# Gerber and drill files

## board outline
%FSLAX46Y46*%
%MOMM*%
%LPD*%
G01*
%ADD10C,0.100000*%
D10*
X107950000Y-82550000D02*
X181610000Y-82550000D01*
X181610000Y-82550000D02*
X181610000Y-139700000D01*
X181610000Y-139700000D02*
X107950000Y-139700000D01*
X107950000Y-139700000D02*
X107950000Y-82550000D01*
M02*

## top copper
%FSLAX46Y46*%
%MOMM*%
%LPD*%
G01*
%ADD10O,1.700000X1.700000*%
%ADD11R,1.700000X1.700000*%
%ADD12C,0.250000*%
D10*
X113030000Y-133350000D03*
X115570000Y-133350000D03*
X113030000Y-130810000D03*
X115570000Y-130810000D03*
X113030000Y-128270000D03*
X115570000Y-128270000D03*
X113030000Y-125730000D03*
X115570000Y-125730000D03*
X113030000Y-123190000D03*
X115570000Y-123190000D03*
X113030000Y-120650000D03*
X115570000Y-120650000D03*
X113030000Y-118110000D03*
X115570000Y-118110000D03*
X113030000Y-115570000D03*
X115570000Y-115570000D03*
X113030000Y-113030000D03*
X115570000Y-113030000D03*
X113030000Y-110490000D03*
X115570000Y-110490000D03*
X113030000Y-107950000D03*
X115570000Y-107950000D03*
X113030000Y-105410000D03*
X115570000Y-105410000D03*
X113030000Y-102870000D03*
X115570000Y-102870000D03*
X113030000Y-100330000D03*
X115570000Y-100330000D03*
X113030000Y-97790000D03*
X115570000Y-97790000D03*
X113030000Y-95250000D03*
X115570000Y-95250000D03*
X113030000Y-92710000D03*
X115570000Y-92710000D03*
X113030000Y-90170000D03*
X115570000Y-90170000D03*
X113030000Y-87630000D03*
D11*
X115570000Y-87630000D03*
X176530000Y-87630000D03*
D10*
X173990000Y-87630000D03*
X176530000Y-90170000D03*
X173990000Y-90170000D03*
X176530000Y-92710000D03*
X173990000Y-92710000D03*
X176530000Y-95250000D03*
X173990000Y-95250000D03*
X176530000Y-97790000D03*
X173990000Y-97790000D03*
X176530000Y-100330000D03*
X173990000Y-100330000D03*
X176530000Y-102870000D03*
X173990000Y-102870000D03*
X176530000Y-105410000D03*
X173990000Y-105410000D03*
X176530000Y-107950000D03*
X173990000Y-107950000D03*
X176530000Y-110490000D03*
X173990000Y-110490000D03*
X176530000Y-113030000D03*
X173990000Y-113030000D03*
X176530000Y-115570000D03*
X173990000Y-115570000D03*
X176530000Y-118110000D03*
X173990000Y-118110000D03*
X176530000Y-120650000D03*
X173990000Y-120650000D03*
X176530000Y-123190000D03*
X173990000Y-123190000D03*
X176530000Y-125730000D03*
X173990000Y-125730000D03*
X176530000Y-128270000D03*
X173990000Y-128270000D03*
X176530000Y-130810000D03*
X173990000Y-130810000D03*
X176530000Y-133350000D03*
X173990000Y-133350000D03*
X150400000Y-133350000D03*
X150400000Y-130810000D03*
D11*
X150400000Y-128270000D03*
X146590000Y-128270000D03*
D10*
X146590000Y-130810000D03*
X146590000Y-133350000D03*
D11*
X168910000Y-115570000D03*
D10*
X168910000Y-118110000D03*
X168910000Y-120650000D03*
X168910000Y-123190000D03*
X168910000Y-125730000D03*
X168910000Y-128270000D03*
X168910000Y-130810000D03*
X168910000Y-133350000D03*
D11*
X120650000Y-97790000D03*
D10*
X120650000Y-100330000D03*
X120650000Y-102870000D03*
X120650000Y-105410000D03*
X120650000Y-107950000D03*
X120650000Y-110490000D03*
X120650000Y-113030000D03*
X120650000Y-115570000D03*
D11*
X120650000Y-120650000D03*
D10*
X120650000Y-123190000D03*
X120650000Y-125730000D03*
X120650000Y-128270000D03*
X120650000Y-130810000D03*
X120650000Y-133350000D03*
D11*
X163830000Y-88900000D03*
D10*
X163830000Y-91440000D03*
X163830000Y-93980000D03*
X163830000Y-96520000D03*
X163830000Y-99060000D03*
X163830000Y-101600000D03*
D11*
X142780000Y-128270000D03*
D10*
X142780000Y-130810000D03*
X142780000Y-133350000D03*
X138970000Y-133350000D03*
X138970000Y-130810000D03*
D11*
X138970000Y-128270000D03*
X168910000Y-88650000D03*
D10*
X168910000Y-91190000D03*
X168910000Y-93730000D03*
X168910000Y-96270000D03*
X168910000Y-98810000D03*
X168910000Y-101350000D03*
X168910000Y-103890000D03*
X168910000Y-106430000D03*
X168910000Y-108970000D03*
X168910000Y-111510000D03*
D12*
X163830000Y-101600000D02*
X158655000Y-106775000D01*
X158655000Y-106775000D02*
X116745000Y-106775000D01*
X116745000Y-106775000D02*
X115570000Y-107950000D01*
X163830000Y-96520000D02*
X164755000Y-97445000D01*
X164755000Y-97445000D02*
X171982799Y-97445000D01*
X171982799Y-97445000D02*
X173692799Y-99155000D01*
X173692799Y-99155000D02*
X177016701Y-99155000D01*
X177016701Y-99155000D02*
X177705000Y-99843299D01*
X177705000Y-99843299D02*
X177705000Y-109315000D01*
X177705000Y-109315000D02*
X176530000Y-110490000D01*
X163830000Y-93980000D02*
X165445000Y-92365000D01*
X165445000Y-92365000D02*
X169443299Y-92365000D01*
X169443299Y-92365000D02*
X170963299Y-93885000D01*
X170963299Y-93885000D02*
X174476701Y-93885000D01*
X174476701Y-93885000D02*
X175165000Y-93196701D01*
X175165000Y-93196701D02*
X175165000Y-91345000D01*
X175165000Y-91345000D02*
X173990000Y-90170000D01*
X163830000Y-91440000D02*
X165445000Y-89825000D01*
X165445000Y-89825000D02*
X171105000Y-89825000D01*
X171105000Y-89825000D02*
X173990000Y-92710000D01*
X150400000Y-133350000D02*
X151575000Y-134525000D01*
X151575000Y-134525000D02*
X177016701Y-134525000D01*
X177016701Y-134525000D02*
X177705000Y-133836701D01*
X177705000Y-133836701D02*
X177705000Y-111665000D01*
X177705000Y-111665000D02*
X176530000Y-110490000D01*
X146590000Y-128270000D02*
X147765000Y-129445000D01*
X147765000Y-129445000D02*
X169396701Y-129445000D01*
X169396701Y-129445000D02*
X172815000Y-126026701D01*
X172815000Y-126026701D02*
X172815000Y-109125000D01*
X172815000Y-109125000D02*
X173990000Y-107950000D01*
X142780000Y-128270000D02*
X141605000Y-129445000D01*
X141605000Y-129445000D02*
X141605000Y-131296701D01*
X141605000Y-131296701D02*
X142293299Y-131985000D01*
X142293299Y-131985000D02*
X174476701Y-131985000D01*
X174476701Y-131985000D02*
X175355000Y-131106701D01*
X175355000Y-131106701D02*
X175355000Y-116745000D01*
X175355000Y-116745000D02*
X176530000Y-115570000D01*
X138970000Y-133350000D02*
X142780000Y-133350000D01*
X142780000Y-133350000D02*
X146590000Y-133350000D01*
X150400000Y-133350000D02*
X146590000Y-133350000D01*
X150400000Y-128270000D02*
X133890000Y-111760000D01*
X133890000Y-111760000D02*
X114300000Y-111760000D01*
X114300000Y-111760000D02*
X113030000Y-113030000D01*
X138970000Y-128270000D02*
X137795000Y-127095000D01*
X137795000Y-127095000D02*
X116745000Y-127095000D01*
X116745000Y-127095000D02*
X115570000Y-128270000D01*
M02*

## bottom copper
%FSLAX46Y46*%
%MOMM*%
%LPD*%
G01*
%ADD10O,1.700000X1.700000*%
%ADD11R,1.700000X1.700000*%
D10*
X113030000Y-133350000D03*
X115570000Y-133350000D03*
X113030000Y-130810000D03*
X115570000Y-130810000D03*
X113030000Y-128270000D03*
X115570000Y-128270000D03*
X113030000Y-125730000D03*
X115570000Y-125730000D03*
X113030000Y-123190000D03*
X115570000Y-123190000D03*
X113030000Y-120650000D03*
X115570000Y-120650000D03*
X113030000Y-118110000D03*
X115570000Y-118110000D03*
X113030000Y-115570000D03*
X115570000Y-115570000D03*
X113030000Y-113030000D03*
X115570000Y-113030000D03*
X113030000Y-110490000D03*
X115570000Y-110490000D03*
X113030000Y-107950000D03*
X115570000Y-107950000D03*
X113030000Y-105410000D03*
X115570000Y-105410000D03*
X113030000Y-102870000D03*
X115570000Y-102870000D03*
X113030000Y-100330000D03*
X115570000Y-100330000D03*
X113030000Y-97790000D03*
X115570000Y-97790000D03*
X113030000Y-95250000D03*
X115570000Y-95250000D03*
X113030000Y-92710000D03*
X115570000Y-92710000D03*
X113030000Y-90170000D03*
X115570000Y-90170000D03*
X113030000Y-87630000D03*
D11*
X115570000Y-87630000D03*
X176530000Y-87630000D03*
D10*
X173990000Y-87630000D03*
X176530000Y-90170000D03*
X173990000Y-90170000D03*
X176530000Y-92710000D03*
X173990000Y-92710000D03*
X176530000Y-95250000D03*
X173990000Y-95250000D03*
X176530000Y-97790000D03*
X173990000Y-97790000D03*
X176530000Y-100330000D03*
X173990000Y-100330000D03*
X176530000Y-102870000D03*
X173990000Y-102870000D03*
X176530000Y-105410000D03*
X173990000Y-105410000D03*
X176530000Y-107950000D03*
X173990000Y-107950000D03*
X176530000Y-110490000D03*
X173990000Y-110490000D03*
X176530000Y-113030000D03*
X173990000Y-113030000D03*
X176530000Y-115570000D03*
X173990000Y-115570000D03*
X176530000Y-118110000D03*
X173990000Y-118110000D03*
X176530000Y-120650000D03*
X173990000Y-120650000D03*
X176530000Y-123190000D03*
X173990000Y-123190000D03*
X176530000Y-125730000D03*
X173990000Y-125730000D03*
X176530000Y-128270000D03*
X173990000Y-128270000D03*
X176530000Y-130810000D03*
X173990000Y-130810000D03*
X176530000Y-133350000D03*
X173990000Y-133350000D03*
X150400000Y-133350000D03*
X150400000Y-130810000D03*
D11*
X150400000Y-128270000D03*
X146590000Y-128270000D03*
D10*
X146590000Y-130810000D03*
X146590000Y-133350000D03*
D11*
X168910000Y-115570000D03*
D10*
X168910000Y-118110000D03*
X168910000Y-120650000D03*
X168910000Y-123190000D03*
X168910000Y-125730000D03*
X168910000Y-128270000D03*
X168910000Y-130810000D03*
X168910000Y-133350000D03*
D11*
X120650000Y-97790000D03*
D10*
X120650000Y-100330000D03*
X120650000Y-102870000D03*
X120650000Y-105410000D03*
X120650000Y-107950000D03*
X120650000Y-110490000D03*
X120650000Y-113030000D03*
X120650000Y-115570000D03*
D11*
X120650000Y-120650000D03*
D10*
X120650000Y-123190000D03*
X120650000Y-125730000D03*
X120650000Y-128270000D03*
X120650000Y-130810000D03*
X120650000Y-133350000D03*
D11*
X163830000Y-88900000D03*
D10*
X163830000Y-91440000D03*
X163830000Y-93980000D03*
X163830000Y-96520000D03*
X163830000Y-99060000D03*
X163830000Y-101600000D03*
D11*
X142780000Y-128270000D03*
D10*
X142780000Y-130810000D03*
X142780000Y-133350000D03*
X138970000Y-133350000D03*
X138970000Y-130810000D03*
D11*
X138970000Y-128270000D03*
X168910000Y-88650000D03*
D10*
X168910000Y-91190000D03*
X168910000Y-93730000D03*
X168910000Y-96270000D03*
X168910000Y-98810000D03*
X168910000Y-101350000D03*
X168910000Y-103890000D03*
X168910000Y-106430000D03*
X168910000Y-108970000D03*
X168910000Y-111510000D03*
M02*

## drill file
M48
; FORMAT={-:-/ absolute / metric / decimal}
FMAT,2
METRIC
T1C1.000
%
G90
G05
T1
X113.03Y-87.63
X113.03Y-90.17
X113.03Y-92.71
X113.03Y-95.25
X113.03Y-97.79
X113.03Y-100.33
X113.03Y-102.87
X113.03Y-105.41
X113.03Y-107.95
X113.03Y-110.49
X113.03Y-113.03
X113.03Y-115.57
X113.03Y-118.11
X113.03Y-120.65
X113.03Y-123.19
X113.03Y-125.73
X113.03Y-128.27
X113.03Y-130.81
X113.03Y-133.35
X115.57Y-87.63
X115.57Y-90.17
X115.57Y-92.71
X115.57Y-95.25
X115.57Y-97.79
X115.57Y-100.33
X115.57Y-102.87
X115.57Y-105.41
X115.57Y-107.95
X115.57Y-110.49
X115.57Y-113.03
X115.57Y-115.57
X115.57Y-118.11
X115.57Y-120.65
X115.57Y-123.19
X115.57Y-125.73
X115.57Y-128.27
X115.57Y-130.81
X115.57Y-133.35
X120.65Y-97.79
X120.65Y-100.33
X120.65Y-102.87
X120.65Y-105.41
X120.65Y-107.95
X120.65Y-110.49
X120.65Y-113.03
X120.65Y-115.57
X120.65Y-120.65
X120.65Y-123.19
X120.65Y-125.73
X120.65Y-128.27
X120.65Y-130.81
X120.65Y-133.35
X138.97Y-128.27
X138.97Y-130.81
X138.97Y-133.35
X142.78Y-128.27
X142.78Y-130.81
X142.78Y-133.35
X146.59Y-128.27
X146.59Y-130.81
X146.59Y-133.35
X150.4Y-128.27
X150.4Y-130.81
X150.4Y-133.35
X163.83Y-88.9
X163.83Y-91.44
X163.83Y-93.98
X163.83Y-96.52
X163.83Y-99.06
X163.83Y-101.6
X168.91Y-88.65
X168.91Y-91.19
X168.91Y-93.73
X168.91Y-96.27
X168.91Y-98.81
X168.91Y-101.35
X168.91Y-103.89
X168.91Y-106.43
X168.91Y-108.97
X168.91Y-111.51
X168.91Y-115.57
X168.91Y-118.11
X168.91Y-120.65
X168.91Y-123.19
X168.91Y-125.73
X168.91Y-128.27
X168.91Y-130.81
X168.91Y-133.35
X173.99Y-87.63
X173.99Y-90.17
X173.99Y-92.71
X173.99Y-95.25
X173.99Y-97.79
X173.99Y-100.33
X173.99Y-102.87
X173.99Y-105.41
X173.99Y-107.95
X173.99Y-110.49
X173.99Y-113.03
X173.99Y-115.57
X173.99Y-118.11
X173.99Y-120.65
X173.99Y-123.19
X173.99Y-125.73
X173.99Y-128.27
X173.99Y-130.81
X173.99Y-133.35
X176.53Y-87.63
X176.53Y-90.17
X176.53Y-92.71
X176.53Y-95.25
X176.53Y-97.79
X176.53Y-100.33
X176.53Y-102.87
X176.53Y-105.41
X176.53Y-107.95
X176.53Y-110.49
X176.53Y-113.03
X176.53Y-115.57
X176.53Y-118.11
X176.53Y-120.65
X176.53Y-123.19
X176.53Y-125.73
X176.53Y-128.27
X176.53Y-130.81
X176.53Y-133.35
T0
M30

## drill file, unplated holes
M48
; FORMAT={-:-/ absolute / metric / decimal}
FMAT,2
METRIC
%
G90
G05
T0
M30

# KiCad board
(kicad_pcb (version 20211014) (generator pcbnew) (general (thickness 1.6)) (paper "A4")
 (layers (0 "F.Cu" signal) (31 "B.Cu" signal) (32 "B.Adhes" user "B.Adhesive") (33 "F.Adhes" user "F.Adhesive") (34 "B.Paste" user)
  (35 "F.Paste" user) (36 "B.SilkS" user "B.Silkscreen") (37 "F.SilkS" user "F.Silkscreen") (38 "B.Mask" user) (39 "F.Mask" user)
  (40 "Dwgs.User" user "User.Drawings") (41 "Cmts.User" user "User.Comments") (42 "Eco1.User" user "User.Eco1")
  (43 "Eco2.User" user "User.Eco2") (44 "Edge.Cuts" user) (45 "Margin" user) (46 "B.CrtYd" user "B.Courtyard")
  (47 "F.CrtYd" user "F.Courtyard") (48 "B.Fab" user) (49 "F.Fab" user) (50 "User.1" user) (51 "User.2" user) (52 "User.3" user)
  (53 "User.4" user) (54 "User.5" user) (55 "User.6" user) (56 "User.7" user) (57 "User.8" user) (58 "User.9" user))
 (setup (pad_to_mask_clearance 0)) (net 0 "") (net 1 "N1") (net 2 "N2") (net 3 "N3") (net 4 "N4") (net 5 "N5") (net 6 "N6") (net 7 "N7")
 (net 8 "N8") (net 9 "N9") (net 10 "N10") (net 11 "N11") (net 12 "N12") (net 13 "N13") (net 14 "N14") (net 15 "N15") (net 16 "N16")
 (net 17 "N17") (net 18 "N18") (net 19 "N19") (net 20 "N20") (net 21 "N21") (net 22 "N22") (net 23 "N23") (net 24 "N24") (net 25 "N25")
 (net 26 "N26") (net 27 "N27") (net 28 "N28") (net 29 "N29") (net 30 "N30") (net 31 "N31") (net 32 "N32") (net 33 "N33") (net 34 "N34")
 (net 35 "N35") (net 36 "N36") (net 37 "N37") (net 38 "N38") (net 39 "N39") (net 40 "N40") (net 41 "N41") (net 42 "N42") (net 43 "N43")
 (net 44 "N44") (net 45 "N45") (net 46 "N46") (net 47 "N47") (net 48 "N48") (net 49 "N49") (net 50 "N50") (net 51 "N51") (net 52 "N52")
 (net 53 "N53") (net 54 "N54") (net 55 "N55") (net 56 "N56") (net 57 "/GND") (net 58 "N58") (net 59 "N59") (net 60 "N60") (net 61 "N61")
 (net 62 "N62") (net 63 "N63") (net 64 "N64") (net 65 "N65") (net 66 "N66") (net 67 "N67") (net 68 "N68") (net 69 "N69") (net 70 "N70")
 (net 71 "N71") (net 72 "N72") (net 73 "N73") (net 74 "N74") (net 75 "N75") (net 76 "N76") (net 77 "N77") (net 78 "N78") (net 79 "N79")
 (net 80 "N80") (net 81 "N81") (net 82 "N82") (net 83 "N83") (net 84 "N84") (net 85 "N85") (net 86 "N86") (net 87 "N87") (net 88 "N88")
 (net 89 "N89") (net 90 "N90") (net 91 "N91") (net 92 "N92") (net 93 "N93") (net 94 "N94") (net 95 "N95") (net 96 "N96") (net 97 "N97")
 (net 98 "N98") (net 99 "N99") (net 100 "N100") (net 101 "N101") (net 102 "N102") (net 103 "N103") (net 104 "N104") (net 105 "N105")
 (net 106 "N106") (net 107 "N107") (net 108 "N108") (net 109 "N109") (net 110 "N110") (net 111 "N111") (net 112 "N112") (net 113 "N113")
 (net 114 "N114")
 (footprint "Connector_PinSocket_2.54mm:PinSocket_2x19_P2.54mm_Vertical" (layer "F.Cu") (at 115.57 87.63)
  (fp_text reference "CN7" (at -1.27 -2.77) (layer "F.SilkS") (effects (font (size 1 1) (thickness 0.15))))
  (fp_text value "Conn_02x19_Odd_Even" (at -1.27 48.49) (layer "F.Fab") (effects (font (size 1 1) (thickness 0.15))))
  (pad "1" thru_hole rect locked (at 0 0) (size 1.7 1.7) (drill 1) (layers *.Cu *.Mask) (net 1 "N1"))
  (pad "2" thru_hole oval locked (at -2.54 0) (size 1.7 1.7) (drill 1) (layers *.Cu *.Mask) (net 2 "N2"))
  (pad "3" thru_hole oval locked (at 0 2.54) (size 1.7 1.7) (drill 1) (layers *.Cu *.Mask) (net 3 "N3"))
  (pad "4" thru_hole oval locked (at -2.54 2.54) (size 1.7 1.7) (drill 1) (layers *.Cu *.Mask) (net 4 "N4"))
  (pad "5" thru_hole oval locked (at 0 5.08) (size 1.7 1.7) (drill 1) (layers *.Cu *.Mask) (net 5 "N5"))
  (pad "6" thru_hole oval locked (at -2.54 5.08) (size 1.7 1.7) (drill 1) (layers *.Cu *.Mask) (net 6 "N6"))
  (pad "7" thru_hole oval locked (at 0 7.62) (size 1.7 1.7) (drill 1) (layers *.Cu *.Mask) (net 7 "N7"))
  (pad "8" thru_hole oval locked (at -2.54 7.62) (size 1.7 1.7) (drill 1) (layers *.Cu *.Mask) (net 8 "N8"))
  (pad "9" thru_hole oval locked (at 0 10.16) (size 1.7 1.7) (drill 1) (layers *.Cu *.Mask) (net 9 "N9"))
  (pad "10" thru_hole oval locked (at -2.54 10.16) (size 1.7 1.7) (drill 1) (layers *.Cu *.Mask) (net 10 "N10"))
  (pad "11" thru_hole oval locked (at 0 12.7) (size 1.7 1.7) (drill 1) (layers *.Cu *.Mask) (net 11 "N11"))
  (pad "12" thru_hole oval locked (at -2.54 12.7) (size 1.7 1.7) (drill 1) (layers *.Cu *.Mask) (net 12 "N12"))
  (pad "13" thru_hole oval locked (at 0 15.24) (size 1.7 1.7) (drill 1) (layers *.Cu *.Mask) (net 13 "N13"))
  (pad "14" thru_hole oval locked (at -2.54 15.24) (size 1.7 1.7) (drill 1) (layers *.Cu *.Mask) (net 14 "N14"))
  (pad "15" thru_hole oval locked (at 0 17.78) (size 1.7 1.7) (drill 1) (layers *.Cu *.Mask) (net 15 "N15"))
  (pad "16" thru_hole oval locked (at -2.54 17.78) (size 1.7 1.7) (drill 1) (layers *.Cu *.Mask) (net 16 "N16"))
  (pad "17" thru_hole oval locked (at 0 20.32) (size 1.7 1.7) (drill 1) (layers *.Cu *.Mask) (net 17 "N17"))
  (pad "18" thru_hole oval locked (at -2.54 20.32) (size 1.7 1.7) (drill 1) (layers *.Cu *.Mask) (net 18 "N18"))
  (pad "19" thru_hole oval locked (at 0 22.86) (size 1.7 1.7) (drill 1) (layers *.Cu *.Mask) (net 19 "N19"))
  (pad "20" thru_hole oval locked (at -2.54 22.86) (size 1.7 1.7) (drill 1) (layers *.Cu *.Mask) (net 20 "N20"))
  (pad "21" thru_hole oval locked (at 0 25.4) (size 1.7 1.7) (drill 1) (layers *.Cu *.Mask) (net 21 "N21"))
  (pad "22" thru_hole oval locked (at -2.54 25.4) (size 1.7 1.7) (drill 1) (layers *.Cu *.Mask) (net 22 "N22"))
  (pad "23" thru_hole oval locked (at 0 27.94) (size 1.7 1.7) (drill 1) (layers *.Cu *.Mask) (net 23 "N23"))
  (pad "24" thru_hole oval locked (at -2.54 27.94) (size 1.7 1.7) (drill 1) (layers *.Cu *.Mask) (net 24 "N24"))
  (pad "25" thru_hole oval locked (at 0 30.48) (size 1.7 1.7) (drill 1) (layers *.Cu *.Mask) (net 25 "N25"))
  (pad "26" thru_hole oval locked (at -2.54 30.48) (size 1.7 1.7) (drill 1) (layers *.Cu *.Mask) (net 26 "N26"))
  (pad "27" thru_hole oval locked (at 0 33.02) (size 1.7 1.7) (drill 1) (layers *.Cu *.Mask) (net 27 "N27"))
  (pad "28" thru_hole oval locked (at -2.54 33.02) (size 1.7 1.7) (drill 1) (layers *.Cu *.Mask) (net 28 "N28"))
  (pad "29" thru_hole oval locked (at 0 35.56) (size 1.7 1.7) (drill 1) (layers *.Cu *.Mask) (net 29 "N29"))
  (pad "30" thru_hole oval locked (at -2.54 35.56) (size 1.7 1.7) (drill 1) (layers *.Cu *.Mask) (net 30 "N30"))
  (pad "31" thru_hole oval locked (at 0 38.1) (size 1.7 1.7) (drill 1) (layers *.Cu *.Mask) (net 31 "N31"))
  (pad "32" thru_hole oval locked (at -2.54 38.1) (size 1.7 1.7) (drill 1) (layers *.Cu *.Mask) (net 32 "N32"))
  (pad "33" thru_hole oval locked (at 0 40.64) (size 1.7 1.7) (drill 1) (layers *.Cu *.Mask) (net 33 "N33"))
  (pad "34" thru_hole oval locked (at -2.54 40.64) (size 1.7 1.7) (drill 1) (layers *.Cu *.Mask) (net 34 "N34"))
  (pad "35" thru_hole oval locked (at 0 43.18) (size 1.7 1.7) (drill 1) (layers *.Cu *.Mask) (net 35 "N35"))
  (pad "36" thru_hole oval locked (at -2.54 43.18) (size 1.7 1.7) (drill 1) (layers *.Cu *.Mask) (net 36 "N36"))
  (pad "37" thru_hole oval locked (at 0 45.72) (size 1.7 1.7) (drill 1) (layers *.Cu *.Mask) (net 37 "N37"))
  (pad "38" thru_hole oval locked (at -2.54 45.72) (size 1.7 1.7) (drill 1) (layers *.Cu *.Mask) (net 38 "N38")))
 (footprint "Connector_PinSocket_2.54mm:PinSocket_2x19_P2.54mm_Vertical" (layer "F.Cu") (at 176.53 87.63)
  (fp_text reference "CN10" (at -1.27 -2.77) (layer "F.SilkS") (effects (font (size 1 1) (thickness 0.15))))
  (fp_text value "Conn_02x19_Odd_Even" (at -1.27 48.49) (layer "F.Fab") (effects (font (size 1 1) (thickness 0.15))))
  (pad "1" thru_hole rect (at 0 0) (size 1.7 1.7) (drill 1) (layers *.Cu *.Mask) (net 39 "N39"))
  (pad "2" thru_hole oval (at -2.54 0) (size 1.7 1.7) (drill 1) (layers *.Cu *.Mask) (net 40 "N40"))
  (pad "3" thru_hole oval (at 0 2.54) (size 1.7 1.7) (drill 1) (layers *.Cu *.Mask) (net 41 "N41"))
  (pad "4" thru_hole oval (at -2.54 2.54) (size 1.7 1.7) (drill 1) (layers *.Cu *.Mask) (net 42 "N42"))
  (pad "5" thru_hole oval (at 0 5.08) (size 1.7 1.7) (drill 1) (layers *.Cu *.Mask) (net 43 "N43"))
  (pad "6" thru_hole oval (at -2.54 5.08) (size 1.7 1.7) (drill 1) (layers *.Cu *.Mask) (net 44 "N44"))
  (pad "7" thru_hole oval (at 0 7.62) (size 1.7 1.7) (drill 1) (layers *.Cu *.Mask) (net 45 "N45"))
  (pad "8" thru_hole oval (at -2.54 7.62) (size 1.7 1.7) (drill 1) (layers *.Cu *.Mask) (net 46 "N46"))
  (pad "9" thru_hole oval (at 0 10.16) (size 1.7 1.7) (drill 1) (layers *.Cu *.Mask) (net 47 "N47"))
  (pad "10" thru_hole oval (at -2.54 10.16) (size 1.7 1.7) (drill 1) (layers *.Cu *.Mask) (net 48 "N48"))
  (pad "11" thru_hole oval (at 0 12.7) (size 1.7 1.7) (drill 1) (layers *.Cu *.Mask) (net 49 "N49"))
  (pad "12" thru_hole oval (at -2.54 12.7) (size 1.7 1.7) (drill 1) (layers *.Cu *.Mask) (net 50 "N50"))
  (pad "13" thru_hole oval (at 0 15.24) (size 1.7 1.7) (drill 1) (layers *.Cu *.Mask) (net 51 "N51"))
  (pad "14" thru_hole oval (at -2.54 15.24) (size 1.7 1.7) (drill 1) (layers *.Cu *.Mask) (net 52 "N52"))
  (pad "15" thru_hole oval (at 0 17.78) (size 1.7 1.7) (drill 1) (layers *.Cu *.Mask) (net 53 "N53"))
  (pad "16" thru_hole oval (at -2.54 17.78) (size 1.7 1.7) (drill 1) (layers *.Cu *.Mask) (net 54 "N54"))
  (pad "17" thru_hole oval (at 0 20.32) (size 1.7 1.7) (drill 1) (layers *.Cu *.Mask) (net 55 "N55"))
  (pad "18" thru_hole oval (at -2.54 20.32) (size 1.7 1.7) (drill 1) (layers *.Cu *.Mask) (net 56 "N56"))
  (pad "19" thru_hole oval (at 0 22.86) (size 1.7 1.7) (drill 1) (layers *.Cu *.Mask) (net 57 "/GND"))
  (pad "20" thru_hole oval (at -2.54 22.86) (size 1.7 1.7) (drill 1) (layers *.Cu *.Mask) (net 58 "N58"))
  (pad "21" thru_hole oval (at 0 25.4) (size 1.7 1.7) (drill 1) (layers *.Cu *.Mask) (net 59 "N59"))
  (pad "22" thru_hole oval (at -2.54 25.4) (size 1.7 1.7) (drill 1) (layers *.Cu *.Mask) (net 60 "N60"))
  (pad "23" thru_hole oval (at 0 27.94) (size 1.7 1.7) (drill 1) (layers *.Cu *.Mask) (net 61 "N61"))
  (pad "24" thru_hole oval (at -2.54 27.94) (size 1.7 1.7) (drill 1) (layers *.Cu *.Mask) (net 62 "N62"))
  (pad "25" thru_hole oval (at 0 30.48) (size 1.7 1.7) (drill 1) (layers *.Cu *.Mask) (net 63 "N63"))
  (pad "26" thru_hole oval (at -2.54 30.48) (size 1.7 1.7) (drill 1) (layers *.Cu *.Mask) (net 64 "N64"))
  (pad "27" thru_hole oval (at 0 33.02) (size 1.7 1.7) (drill 1) (layers *.Cu *.Mask) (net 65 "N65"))
  (pad "28" thru_hole oval (at -2.54 33.02) (size 1.7 1.7) (drill 1) (layers *.Cu *.Mask) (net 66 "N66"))
  (pad "29" thru_hole oval (at 0 35.56) (size 1.7 1.7) (drill 1) (layers *.Cu *.Mask) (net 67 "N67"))
  (pad "30" thru_hole oval (at -2.54 35.56) (size 1.7 1.7) (drill 1) (layers *.Cu *.Mask) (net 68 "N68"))
  (pad "31" thru_hole oval (at 0 38.1) (size 1.7 1.7) (drill 1) (layers *.Cu *.Mask) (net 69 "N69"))
  (pad "32" thru_hole oval (at -2.54 38.1) (size 1.7 1.7) (drill 1) (layers *.Cu *.Mask) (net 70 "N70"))
  (pad "33" thru_hole oval (at 0 40.64) (size 1.7 1.7) (drill 1) (layers *.Cu *.Mask) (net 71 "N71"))
  (pad "34" thru_hole oval (at -2.54 40.64) (size 1.7 1.7) (drill 1) (layers *.Cu *.Mask) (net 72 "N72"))
  (pad "35" thru_hole oval (at 0 43.18) (size 1.7 1.7) (drill 1) (layers *.Cu *.Mask) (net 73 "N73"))
  (pad "36" thru_hole oval (at -2.54 43.18) (size 1.7 1.7) (drill 1) (layers *.Cu *.Mask) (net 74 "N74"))
  (pad "37" thru_hole oval (at 0 45.72) (size 1.7 1.7) (drill 1) (layers *.Cu *.Mask) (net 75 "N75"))
  (pad "38" thru_hole oval (at -2.54 45.72) (size 1.7 1.7) (drill 1) (layers *.Cu *.Mask) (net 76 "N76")))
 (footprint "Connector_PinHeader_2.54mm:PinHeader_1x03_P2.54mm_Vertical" (layer "F.Cu") (at 150.4 128.27)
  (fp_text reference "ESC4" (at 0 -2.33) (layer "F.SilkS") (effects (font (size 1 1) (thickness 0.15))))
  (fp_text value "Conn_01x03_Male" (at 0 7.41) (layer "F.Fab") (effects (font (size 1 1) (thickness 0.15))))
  (pad "1" thru_hole rect (at 0 0) (size 1.7 1.7) (drill 1) (layers *.Cu *.Mask) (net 22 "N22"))
  (pad "2" thru_hole oval (at 0 2.54) (size 1.7 1.7) (drill 1) (layers *.Cu *.Mask) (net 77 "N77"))
  (pad "3" thru_hole oval (at 0 5.08) (size 1.7 1.7) (drill 1) (layers *.Cu *.Mask) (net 57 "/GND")))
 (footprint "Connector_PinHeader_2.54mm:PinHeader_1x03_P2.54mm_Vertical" (layer "F.Cu") (at 146.59 128.27)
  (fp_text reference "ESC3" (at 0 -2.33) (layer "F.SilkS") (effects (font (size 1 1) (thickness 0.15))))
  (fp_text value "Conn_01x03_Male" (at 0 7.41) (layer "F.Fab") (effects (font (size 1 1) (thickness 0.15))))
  (pad "1" thru_hole rect (at 0 0) (size 1.7 1.7) (drill 1) (layers *.Cu *.Mask) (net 56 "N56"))
  (pad "2" thru_hole oval (at 0 2.54) (size 1.7 1.7) (drill 1) (layers *.Cu *.Mask) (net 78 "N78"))
  (pad "3" thru_hole oval (at 0 5.08) (size 1.7 1.7) (drill 1) (layers *.Cu *.Mask) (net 57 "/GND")))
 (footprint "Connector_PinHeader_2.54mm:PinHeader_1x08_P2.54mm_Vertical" (layer "F.Cu") (at 168.91 115.57)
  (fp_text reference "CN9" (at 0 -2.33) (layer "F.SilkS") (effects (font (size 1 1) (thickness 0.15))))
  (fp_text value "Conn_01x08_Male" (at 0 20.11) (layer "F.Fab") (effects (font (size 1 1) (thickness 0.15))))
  (pad "1" thru_hole rect (at 0 0) (size 1.7 1.7) (drill 1) (layers *.Cu *.Mask) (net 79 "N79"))
  (pad "2" thru_hole oval (at 0 2.54) (size 1.7 1.7) (drill 1) (layers *.Cu *.Mask) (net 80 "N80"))
  (pad "3" thru_hole oval (at 0 5.08) (size 1.7 1.7) (drill 1) (layers *.Cu *.Mask) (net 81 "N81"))
  (pad "4" thru_hole oval (at 0 7.62) (size 1.7 1.7) (drill 1) (layers *.Cu *.Mask) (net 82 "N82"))
  (pad "5" thru_hole oval (at 0 10.16) (size 1.7 1.7) (drill 1) (layers *.Cu *.Mask) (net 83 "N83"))
  (pad "6" thru_hole oval (at 0 12.7) (size 1.7 1.7) (drill 1) (layers *.Cu *.Mask) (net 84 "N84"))
  (pad "7" thru_hole oval (at 0 15.24) (size 1.7 1.7) (drill 1) (layers *.Cu *.Mask) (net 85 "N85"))
  (pad "8" thru_hole oval (at 0 17.78) (size 1.7 1.7) (drill 1) (layers *.Cu *.Mask) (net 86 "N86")))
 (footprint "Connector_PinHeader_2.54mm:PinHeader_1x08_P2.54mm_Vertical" (layer "F.Cu") (at 120.65 97.79)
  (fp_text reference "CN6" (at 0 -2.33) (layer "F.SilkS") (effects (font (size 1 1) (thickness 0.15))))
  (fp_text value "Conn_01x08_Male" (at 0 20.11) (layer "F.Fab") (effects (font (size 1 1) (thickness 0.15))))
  (pad "1" thru_hole rect (at 0 0) (size 1.7 1.7) (drill 1) (layers *.Cu *.Mask) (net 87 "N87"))
  (pad "2" thru_hole oval (at 0 2.54) (size 1.7 1.7) (drill 1) (layers *.Cu *.Mask) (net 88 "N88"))
  (pad "3" thru_hole oval (at 0 5.08) (size 1.7 1.7) (drill 1) (layers *.Cu *.Mask) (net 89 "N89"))
  (pad "4" thru_hole oval (at 0 7.62) (size 1.7 1.7) (drill 1) (layers *.Cu *.Mask) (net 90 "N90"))
  (pad "5" thru_hole oval (at 0 10.16) (size 1.7 1.7) (drill 1) (layers *.Cu *.Mask) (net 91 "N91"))
  (pad "6" thru_hole oval (at 0 12.7) (size 1.7 1.7) (drill 1) (layers *.Cu *.Mask) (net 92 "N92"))
  (pad "7" thru_hole oval (at 0 15.24) (size 1.7 1.7) (drill 1) (layers *.Cu *.Mask) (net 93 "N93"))
  (pad "8" thru_hole oval (at 0 17.78) (size 1.7 1.7) (drill 1) (layers *.Cu *.Mask) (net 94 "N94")))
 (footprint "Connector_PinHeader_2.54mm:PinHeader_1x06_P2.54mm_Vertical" (layer "F.Cu") (at 120.65 120.65)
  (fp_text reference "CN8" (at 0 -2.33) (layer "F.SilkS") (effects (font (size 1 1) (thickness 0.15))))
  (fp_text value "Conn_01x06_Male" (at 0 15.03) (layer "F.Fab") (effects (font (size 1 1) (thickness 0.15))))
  (pad "1" thru_hole rect (at 0 0) (size 1.7 1.7) (drill 1) (layers *.Cu *.Mask) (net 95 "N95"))
  (pad "2" thru_hole oval (at 0 2.54) (size 1.7 1.7) (drill 1) (layers *.Cu *.Mask) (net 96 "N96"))
  (pad "3" thru_hole oval (at 0 5.08) (size 1.7 1.7) (drill 1) (layers *.Cu *.Mask) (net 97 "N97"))
  (pad "4" thru_hole oval (at 0 7.62) (size 1.7 1.7) (drill 1) (layers *.Cu *.Mask) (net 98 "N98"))
  (pad "5" thru_hole oval (at 0 10.16) (size 1.7 1.7) (drill 1) (layers *.Cu *.Mask) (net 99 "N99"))
  (pad "6" thru_hole oval (at 0 12.7) (size 1.7 1.7) (drill 1) (layers *.Cu *.Mask) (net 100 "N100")))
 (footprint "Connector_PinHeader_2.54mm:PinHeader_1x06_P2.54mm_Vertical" (layer "F.Cu") (at 163.83 88.9)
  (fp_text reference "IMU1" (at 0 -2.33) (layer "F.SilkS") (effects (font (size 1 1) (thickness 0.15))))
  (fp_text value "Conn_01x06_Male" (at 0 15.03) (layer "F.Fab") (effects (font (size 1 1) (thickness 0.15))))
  (pad "1" thru_hole rect (at 0 0) (size 1.7 1.7) (drill 1) (layers *.Cu *.Mask) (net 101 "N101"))
  (pad "2" thru_hole oval (at 0 2.54) (size 1.7 1.7) (drill 1) (layers *.Cu *.Mask) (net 44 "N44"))
  (pad "3" thru_hole oval (at 0 5.08) (size 1.7 1.7) (drill 1) (layers *.Cu *.Mask) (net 42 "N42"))
  (pad "4" thru_hole oval (at 0 7.62) (size 1.7 1.7) (drill 1) (layers *.Cu *.Mask) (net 57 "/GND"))
  (pad "5" thru_hole oval (at 0 10.16) (size 1.7 1.7) (drill 1) (layers *.Cu *.Mask) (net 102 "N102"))
  (pad "6" thru_hole oval (at 0 12.7) (size 1.7 1.7) (drill 1) (layers *.Cu *.Mask) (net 17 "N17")))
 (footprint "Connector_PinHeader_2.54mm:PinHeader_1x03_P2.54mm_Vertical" (layer "F.Cu") (at 142.78 128.27)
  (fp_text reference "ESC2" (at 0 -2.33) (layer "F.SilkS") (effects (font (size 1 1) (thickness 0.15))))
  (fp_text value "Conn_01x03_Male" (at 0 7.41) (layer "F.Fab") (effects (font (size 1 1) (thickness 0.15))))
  (pad "1" thru_hole rect (at 0 0) (size 1.7 1.7) (drill 1) (layers *.Cu *.Mask) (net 61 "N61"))
  (pad "2" thru_hole oval (at 0 2.54) (size 1.7 1.7) (drill 1) (layers *.Cu *.Mask) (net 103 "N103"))
  (pad "3" thru_hole oval (at 0 5.08) (size 1.7 1.7) (drill 1) (layers *.Cu *.Mask) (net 57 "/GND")))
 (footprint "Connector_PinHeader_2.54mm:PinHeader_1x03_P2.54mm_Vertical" (layer "F.Cu") (at 138.97 128.27)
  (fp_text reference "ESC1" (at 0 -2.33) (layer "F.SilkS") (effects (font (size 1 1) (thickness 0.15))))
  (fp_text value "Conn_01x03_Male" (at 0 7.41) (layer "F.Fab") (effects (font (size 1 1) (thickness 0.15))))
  (pad "1" thru_hole rect (at 0 0) (size 1.7 1.7) (drill 1) (layers *.Cu *.Mask) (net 33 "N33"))
  (pad "2" thru_hole oval (at 0 2.54) (size 1.7 1.7) (drill 1) (layers *.Cu *.Mask) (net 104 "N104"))
  (pad "3" thru_hole oval (at 0 5.08) (size 1.7 1.7) (drill 1) (layers *.Cu *.Mask) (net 57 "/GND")))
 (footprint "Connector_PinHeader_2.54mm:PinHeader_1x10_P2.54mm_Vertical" (layer "F.Cu") (at 168.91 88.65)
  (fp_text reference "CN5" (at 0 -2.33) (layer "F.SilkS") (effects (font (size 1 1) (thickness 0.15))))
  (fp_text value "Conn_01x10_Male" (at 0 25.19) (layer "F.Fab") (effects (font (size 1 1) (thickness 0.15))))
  (pad "1" thru_hole rect (at 0 0) (size 1.7 1.7) (drill 1) (layers *.Cu *.Mask) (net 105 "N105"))
  (pad "2" thru_hole oval (at 0 2.54) (size 1.7 1.7) (drill 1) (layers *.Cu *.Mask) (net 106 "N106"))
  (pad "3" thru_hole oval (at 0 5.08) (size 1.7 1.7) (drill 1) (layers *.Cu *.Mask) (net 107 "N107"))
  (pad "4" thru_hole oval (at 0 7.62) (size 1.7 1.7) (drill 1) (layers *.Cu *.Mask) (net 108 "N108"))
  (pad "5" thru_hole oval (at 0 10.16) (size 1.7 1.7) (drill 1) (layers *.Cu *.Mask) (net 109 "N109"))
  (pad "6" thru_hole oval (at 0 12.7) (size 1.7 1.7) (drill 1) (layers *.Cu *.Mask) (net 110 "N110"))
  (pad "7" thru_hole oval (at 0 15.24) (size 1.7 1.7) (drill 1) (layers *.Cu *.Mask) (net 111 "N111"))
  (pad "8" thru_hole oval (at 0 17.78) (size 1.7 1.7) (drill 1) (layers *.Cu *.Mask) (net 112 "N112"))
  (pad "9" thru_hole oval (at 0 20.32) (size 1.7 1.7) (drill 1) (layers *.Cu *.Mask) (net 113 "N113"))
  (pad "10" thru_hole oval (at 0 22.86) (size 1.7 1.7) (drill 1) (layers *.Cu *.Mask) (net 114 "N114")))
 (gr_rect (start 107.95 82.55) (end 181.61 139.7) (layer "Edge.Cuts") (width 0.1) (fill none))
 (segment (start 133.89 111.76) (end 114.3 111.76) (width 0.25) (layer "F.Cu") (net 22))
 (segment (start 150.4 128.27) (end 133.89 111.76) (width 0.25) (layer "F.Cu") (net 22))
 (segment (start 114.3 111.76) (end 113.03 113.03) (width 0.25) (layer "F.Cu") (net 22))
 (segment (start 177.016701 99.155) (end 177.705 99.843299) (width 0.25) (layer "F.Cu") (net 57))
 (segment (start 177.705 99.843299) (end 177.705 109.315) (width 0.25) (layer "F.Cu") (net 57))
 (segment (start 177.705 111.665) (end 176.53 110.49) (width 0.25) (layer "F.Cu") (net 57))
 (segment (start 138.97 133.35) (end 142.78 133.35) (width 0.25) (layer "F.Cu") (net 57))
 (segment (start 173.692799 99.155) (end 177.016701 99.155) (width 0.25) (layer "F.Cu") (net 57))
 (segment (start 150.4 133.35) (end 151.575 134.525) (width 0.25) (layer "F.Cu") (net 57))
 (segment (start 177.705 109.315) (end 176.53 110.49) (width 0.25) (layer "F.Cu") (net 57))
 (segment (start 150.4 133.35) (end 146.59 133.35) (width 0.25) (layer "F.Cu") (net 57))
 (segment (start 163.83 96.52) (end 164.755 97.445) (width 0.25) (layer "F.Cu") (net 57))
 (segment (start 177.705 133.836701) (end 177.705 111.665) (width 0.25) (layer "F.Cu") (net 57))
 (segment (start 151.575 134.525) (end 177.016701 134.525) (width 0.25) (layer "F.Cu") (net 57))
 (segment (start 142.78 133.35) (end 146.59 133.35) (width 0.25) (layer "F.Cu") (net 57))
 (segment (start 177.016701 134.525) (end 177.705 133.836701) (width 0.25) (layer "F.Cu") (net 57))
 (segment (start 164.755 97.445) (end 171.982799 97.445) (width 0.25) (layer "F.Cu") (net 57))
 (segment (start 171.982799 97.445) (end 173.692799 99.155) (width 0.25) (layer "F.Cu") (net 57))
 (segment (start 138.97 128.27) (end 137.795 127.095) (width 0.25) (layer "F.Cu") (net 33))
 (segment (start 137.795 127.095) (end 116.745 127.095) (width 0.25) (layer "F.Cu") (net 33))
 (segment (start 116.745 127.095) (end 115.57 128.27) (width 0.25) (layer "F.Cu") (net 33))
 (segment (start 158.655 106.775) (end 116.745 106.775) (width 0.25) (layer "F.Cu") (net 17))
 (segment (start 116.745 106.775) (end 115.57 107.95) (width 0.25) (layer "F.Cu") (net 17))
 (segment (start 163.83 101.6) (end 158.655 106.775) (width 0.25) (layer "F.Cu") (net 17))
 (segment (start 175.165 93.196701) (end 175.165 91.345) (width 0.25) (layer "F.Cu") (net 42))
 (segment (start 170.963299 93.885) (end 174.476701 93.885) (width 0.25) (layer "F.Cu") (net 42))
 (segment (start 169.443299 92.365) (end 170.963299 93.885) (width 0.25) (layer "F.Cu") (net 42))
 (segment (start 163.83 93.98) (end 165.445 92.365) (width 0.25) (layer "F.Cu") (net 42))
 (segment (start 174.476701 93.885) (end 175.165 93.196701) (width 0.25) (layer "F.Cu") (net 42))
 (segment (start 165.445 92.365) (end 169.443299 92.365) (width 0.25) (layer "F.Cu") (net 42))
 (segment (start 175.165 91.345) (end 173.99 90.17) (width 0.25) (layer "F.Cu") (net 42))
 (segment (start 165.445 89.825) (end 171.105 89.825) (width 0.25) (layer "F.Cu") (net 44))
 (segment (start 171.105 89.825) (end 173.99 92.71) (width 0.25) (layer "F.Cu") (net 44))
 (segment (start 163.83 91.44) (end 165.445 89.825) (width 0.25) (layer "F.Cu") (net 44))
 (segment (start 146.59 128.27) (end 147.765 129.445) (width 0.25) (layer "F.Cu") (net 56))
 (segment (start 172.815 109.125) (end 173.99 107.95) (width 0.25) (layer "F.Cu") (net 56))
 (segment (start 147.765 129.445) (end 169.396701 129.445) (width 0.25) (layer "F.Cu") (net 56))
 (segment (start 169.396701 129.445) (end 172.815 126.026701) (width 0.25) (layer "F.Cu") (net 56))
 (segment (start 172.815 126.026701) (end 172.815 109.125) (width 0.25) (layer "F.Cu") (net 56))
 (segment (start 175.355 116.745) (end 176.53 115.57) (width 0.25) (layer "F.Cu") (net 61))
 (segment (start 141.605 131.296701) (end 142.293299 131.985) (width 0.25) (layer "F.Cu") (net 61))
 (segment (start 141.605 129.445) (end 141.605 131.296701) (width 0.25) (layer "F.Cu") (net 61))
 (segment (start 174.476701 131.985) (end 175.355 131.106701) (width 0.25) (layer "F.Cu") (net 61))
 (segment (start 142.293299 131.985) (end 174.476701 131.985) (width 0.25) (layer "F.Cu") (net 61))
 (segment (start 175.355 131.106701) (end 175.355 116.745) (width 0.25) (layer "F.Cu") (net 61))
 (segment (start 142.78 128.27) (end 141.605 129.445) (width 0.25) (layer "F.Cu") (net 61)))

